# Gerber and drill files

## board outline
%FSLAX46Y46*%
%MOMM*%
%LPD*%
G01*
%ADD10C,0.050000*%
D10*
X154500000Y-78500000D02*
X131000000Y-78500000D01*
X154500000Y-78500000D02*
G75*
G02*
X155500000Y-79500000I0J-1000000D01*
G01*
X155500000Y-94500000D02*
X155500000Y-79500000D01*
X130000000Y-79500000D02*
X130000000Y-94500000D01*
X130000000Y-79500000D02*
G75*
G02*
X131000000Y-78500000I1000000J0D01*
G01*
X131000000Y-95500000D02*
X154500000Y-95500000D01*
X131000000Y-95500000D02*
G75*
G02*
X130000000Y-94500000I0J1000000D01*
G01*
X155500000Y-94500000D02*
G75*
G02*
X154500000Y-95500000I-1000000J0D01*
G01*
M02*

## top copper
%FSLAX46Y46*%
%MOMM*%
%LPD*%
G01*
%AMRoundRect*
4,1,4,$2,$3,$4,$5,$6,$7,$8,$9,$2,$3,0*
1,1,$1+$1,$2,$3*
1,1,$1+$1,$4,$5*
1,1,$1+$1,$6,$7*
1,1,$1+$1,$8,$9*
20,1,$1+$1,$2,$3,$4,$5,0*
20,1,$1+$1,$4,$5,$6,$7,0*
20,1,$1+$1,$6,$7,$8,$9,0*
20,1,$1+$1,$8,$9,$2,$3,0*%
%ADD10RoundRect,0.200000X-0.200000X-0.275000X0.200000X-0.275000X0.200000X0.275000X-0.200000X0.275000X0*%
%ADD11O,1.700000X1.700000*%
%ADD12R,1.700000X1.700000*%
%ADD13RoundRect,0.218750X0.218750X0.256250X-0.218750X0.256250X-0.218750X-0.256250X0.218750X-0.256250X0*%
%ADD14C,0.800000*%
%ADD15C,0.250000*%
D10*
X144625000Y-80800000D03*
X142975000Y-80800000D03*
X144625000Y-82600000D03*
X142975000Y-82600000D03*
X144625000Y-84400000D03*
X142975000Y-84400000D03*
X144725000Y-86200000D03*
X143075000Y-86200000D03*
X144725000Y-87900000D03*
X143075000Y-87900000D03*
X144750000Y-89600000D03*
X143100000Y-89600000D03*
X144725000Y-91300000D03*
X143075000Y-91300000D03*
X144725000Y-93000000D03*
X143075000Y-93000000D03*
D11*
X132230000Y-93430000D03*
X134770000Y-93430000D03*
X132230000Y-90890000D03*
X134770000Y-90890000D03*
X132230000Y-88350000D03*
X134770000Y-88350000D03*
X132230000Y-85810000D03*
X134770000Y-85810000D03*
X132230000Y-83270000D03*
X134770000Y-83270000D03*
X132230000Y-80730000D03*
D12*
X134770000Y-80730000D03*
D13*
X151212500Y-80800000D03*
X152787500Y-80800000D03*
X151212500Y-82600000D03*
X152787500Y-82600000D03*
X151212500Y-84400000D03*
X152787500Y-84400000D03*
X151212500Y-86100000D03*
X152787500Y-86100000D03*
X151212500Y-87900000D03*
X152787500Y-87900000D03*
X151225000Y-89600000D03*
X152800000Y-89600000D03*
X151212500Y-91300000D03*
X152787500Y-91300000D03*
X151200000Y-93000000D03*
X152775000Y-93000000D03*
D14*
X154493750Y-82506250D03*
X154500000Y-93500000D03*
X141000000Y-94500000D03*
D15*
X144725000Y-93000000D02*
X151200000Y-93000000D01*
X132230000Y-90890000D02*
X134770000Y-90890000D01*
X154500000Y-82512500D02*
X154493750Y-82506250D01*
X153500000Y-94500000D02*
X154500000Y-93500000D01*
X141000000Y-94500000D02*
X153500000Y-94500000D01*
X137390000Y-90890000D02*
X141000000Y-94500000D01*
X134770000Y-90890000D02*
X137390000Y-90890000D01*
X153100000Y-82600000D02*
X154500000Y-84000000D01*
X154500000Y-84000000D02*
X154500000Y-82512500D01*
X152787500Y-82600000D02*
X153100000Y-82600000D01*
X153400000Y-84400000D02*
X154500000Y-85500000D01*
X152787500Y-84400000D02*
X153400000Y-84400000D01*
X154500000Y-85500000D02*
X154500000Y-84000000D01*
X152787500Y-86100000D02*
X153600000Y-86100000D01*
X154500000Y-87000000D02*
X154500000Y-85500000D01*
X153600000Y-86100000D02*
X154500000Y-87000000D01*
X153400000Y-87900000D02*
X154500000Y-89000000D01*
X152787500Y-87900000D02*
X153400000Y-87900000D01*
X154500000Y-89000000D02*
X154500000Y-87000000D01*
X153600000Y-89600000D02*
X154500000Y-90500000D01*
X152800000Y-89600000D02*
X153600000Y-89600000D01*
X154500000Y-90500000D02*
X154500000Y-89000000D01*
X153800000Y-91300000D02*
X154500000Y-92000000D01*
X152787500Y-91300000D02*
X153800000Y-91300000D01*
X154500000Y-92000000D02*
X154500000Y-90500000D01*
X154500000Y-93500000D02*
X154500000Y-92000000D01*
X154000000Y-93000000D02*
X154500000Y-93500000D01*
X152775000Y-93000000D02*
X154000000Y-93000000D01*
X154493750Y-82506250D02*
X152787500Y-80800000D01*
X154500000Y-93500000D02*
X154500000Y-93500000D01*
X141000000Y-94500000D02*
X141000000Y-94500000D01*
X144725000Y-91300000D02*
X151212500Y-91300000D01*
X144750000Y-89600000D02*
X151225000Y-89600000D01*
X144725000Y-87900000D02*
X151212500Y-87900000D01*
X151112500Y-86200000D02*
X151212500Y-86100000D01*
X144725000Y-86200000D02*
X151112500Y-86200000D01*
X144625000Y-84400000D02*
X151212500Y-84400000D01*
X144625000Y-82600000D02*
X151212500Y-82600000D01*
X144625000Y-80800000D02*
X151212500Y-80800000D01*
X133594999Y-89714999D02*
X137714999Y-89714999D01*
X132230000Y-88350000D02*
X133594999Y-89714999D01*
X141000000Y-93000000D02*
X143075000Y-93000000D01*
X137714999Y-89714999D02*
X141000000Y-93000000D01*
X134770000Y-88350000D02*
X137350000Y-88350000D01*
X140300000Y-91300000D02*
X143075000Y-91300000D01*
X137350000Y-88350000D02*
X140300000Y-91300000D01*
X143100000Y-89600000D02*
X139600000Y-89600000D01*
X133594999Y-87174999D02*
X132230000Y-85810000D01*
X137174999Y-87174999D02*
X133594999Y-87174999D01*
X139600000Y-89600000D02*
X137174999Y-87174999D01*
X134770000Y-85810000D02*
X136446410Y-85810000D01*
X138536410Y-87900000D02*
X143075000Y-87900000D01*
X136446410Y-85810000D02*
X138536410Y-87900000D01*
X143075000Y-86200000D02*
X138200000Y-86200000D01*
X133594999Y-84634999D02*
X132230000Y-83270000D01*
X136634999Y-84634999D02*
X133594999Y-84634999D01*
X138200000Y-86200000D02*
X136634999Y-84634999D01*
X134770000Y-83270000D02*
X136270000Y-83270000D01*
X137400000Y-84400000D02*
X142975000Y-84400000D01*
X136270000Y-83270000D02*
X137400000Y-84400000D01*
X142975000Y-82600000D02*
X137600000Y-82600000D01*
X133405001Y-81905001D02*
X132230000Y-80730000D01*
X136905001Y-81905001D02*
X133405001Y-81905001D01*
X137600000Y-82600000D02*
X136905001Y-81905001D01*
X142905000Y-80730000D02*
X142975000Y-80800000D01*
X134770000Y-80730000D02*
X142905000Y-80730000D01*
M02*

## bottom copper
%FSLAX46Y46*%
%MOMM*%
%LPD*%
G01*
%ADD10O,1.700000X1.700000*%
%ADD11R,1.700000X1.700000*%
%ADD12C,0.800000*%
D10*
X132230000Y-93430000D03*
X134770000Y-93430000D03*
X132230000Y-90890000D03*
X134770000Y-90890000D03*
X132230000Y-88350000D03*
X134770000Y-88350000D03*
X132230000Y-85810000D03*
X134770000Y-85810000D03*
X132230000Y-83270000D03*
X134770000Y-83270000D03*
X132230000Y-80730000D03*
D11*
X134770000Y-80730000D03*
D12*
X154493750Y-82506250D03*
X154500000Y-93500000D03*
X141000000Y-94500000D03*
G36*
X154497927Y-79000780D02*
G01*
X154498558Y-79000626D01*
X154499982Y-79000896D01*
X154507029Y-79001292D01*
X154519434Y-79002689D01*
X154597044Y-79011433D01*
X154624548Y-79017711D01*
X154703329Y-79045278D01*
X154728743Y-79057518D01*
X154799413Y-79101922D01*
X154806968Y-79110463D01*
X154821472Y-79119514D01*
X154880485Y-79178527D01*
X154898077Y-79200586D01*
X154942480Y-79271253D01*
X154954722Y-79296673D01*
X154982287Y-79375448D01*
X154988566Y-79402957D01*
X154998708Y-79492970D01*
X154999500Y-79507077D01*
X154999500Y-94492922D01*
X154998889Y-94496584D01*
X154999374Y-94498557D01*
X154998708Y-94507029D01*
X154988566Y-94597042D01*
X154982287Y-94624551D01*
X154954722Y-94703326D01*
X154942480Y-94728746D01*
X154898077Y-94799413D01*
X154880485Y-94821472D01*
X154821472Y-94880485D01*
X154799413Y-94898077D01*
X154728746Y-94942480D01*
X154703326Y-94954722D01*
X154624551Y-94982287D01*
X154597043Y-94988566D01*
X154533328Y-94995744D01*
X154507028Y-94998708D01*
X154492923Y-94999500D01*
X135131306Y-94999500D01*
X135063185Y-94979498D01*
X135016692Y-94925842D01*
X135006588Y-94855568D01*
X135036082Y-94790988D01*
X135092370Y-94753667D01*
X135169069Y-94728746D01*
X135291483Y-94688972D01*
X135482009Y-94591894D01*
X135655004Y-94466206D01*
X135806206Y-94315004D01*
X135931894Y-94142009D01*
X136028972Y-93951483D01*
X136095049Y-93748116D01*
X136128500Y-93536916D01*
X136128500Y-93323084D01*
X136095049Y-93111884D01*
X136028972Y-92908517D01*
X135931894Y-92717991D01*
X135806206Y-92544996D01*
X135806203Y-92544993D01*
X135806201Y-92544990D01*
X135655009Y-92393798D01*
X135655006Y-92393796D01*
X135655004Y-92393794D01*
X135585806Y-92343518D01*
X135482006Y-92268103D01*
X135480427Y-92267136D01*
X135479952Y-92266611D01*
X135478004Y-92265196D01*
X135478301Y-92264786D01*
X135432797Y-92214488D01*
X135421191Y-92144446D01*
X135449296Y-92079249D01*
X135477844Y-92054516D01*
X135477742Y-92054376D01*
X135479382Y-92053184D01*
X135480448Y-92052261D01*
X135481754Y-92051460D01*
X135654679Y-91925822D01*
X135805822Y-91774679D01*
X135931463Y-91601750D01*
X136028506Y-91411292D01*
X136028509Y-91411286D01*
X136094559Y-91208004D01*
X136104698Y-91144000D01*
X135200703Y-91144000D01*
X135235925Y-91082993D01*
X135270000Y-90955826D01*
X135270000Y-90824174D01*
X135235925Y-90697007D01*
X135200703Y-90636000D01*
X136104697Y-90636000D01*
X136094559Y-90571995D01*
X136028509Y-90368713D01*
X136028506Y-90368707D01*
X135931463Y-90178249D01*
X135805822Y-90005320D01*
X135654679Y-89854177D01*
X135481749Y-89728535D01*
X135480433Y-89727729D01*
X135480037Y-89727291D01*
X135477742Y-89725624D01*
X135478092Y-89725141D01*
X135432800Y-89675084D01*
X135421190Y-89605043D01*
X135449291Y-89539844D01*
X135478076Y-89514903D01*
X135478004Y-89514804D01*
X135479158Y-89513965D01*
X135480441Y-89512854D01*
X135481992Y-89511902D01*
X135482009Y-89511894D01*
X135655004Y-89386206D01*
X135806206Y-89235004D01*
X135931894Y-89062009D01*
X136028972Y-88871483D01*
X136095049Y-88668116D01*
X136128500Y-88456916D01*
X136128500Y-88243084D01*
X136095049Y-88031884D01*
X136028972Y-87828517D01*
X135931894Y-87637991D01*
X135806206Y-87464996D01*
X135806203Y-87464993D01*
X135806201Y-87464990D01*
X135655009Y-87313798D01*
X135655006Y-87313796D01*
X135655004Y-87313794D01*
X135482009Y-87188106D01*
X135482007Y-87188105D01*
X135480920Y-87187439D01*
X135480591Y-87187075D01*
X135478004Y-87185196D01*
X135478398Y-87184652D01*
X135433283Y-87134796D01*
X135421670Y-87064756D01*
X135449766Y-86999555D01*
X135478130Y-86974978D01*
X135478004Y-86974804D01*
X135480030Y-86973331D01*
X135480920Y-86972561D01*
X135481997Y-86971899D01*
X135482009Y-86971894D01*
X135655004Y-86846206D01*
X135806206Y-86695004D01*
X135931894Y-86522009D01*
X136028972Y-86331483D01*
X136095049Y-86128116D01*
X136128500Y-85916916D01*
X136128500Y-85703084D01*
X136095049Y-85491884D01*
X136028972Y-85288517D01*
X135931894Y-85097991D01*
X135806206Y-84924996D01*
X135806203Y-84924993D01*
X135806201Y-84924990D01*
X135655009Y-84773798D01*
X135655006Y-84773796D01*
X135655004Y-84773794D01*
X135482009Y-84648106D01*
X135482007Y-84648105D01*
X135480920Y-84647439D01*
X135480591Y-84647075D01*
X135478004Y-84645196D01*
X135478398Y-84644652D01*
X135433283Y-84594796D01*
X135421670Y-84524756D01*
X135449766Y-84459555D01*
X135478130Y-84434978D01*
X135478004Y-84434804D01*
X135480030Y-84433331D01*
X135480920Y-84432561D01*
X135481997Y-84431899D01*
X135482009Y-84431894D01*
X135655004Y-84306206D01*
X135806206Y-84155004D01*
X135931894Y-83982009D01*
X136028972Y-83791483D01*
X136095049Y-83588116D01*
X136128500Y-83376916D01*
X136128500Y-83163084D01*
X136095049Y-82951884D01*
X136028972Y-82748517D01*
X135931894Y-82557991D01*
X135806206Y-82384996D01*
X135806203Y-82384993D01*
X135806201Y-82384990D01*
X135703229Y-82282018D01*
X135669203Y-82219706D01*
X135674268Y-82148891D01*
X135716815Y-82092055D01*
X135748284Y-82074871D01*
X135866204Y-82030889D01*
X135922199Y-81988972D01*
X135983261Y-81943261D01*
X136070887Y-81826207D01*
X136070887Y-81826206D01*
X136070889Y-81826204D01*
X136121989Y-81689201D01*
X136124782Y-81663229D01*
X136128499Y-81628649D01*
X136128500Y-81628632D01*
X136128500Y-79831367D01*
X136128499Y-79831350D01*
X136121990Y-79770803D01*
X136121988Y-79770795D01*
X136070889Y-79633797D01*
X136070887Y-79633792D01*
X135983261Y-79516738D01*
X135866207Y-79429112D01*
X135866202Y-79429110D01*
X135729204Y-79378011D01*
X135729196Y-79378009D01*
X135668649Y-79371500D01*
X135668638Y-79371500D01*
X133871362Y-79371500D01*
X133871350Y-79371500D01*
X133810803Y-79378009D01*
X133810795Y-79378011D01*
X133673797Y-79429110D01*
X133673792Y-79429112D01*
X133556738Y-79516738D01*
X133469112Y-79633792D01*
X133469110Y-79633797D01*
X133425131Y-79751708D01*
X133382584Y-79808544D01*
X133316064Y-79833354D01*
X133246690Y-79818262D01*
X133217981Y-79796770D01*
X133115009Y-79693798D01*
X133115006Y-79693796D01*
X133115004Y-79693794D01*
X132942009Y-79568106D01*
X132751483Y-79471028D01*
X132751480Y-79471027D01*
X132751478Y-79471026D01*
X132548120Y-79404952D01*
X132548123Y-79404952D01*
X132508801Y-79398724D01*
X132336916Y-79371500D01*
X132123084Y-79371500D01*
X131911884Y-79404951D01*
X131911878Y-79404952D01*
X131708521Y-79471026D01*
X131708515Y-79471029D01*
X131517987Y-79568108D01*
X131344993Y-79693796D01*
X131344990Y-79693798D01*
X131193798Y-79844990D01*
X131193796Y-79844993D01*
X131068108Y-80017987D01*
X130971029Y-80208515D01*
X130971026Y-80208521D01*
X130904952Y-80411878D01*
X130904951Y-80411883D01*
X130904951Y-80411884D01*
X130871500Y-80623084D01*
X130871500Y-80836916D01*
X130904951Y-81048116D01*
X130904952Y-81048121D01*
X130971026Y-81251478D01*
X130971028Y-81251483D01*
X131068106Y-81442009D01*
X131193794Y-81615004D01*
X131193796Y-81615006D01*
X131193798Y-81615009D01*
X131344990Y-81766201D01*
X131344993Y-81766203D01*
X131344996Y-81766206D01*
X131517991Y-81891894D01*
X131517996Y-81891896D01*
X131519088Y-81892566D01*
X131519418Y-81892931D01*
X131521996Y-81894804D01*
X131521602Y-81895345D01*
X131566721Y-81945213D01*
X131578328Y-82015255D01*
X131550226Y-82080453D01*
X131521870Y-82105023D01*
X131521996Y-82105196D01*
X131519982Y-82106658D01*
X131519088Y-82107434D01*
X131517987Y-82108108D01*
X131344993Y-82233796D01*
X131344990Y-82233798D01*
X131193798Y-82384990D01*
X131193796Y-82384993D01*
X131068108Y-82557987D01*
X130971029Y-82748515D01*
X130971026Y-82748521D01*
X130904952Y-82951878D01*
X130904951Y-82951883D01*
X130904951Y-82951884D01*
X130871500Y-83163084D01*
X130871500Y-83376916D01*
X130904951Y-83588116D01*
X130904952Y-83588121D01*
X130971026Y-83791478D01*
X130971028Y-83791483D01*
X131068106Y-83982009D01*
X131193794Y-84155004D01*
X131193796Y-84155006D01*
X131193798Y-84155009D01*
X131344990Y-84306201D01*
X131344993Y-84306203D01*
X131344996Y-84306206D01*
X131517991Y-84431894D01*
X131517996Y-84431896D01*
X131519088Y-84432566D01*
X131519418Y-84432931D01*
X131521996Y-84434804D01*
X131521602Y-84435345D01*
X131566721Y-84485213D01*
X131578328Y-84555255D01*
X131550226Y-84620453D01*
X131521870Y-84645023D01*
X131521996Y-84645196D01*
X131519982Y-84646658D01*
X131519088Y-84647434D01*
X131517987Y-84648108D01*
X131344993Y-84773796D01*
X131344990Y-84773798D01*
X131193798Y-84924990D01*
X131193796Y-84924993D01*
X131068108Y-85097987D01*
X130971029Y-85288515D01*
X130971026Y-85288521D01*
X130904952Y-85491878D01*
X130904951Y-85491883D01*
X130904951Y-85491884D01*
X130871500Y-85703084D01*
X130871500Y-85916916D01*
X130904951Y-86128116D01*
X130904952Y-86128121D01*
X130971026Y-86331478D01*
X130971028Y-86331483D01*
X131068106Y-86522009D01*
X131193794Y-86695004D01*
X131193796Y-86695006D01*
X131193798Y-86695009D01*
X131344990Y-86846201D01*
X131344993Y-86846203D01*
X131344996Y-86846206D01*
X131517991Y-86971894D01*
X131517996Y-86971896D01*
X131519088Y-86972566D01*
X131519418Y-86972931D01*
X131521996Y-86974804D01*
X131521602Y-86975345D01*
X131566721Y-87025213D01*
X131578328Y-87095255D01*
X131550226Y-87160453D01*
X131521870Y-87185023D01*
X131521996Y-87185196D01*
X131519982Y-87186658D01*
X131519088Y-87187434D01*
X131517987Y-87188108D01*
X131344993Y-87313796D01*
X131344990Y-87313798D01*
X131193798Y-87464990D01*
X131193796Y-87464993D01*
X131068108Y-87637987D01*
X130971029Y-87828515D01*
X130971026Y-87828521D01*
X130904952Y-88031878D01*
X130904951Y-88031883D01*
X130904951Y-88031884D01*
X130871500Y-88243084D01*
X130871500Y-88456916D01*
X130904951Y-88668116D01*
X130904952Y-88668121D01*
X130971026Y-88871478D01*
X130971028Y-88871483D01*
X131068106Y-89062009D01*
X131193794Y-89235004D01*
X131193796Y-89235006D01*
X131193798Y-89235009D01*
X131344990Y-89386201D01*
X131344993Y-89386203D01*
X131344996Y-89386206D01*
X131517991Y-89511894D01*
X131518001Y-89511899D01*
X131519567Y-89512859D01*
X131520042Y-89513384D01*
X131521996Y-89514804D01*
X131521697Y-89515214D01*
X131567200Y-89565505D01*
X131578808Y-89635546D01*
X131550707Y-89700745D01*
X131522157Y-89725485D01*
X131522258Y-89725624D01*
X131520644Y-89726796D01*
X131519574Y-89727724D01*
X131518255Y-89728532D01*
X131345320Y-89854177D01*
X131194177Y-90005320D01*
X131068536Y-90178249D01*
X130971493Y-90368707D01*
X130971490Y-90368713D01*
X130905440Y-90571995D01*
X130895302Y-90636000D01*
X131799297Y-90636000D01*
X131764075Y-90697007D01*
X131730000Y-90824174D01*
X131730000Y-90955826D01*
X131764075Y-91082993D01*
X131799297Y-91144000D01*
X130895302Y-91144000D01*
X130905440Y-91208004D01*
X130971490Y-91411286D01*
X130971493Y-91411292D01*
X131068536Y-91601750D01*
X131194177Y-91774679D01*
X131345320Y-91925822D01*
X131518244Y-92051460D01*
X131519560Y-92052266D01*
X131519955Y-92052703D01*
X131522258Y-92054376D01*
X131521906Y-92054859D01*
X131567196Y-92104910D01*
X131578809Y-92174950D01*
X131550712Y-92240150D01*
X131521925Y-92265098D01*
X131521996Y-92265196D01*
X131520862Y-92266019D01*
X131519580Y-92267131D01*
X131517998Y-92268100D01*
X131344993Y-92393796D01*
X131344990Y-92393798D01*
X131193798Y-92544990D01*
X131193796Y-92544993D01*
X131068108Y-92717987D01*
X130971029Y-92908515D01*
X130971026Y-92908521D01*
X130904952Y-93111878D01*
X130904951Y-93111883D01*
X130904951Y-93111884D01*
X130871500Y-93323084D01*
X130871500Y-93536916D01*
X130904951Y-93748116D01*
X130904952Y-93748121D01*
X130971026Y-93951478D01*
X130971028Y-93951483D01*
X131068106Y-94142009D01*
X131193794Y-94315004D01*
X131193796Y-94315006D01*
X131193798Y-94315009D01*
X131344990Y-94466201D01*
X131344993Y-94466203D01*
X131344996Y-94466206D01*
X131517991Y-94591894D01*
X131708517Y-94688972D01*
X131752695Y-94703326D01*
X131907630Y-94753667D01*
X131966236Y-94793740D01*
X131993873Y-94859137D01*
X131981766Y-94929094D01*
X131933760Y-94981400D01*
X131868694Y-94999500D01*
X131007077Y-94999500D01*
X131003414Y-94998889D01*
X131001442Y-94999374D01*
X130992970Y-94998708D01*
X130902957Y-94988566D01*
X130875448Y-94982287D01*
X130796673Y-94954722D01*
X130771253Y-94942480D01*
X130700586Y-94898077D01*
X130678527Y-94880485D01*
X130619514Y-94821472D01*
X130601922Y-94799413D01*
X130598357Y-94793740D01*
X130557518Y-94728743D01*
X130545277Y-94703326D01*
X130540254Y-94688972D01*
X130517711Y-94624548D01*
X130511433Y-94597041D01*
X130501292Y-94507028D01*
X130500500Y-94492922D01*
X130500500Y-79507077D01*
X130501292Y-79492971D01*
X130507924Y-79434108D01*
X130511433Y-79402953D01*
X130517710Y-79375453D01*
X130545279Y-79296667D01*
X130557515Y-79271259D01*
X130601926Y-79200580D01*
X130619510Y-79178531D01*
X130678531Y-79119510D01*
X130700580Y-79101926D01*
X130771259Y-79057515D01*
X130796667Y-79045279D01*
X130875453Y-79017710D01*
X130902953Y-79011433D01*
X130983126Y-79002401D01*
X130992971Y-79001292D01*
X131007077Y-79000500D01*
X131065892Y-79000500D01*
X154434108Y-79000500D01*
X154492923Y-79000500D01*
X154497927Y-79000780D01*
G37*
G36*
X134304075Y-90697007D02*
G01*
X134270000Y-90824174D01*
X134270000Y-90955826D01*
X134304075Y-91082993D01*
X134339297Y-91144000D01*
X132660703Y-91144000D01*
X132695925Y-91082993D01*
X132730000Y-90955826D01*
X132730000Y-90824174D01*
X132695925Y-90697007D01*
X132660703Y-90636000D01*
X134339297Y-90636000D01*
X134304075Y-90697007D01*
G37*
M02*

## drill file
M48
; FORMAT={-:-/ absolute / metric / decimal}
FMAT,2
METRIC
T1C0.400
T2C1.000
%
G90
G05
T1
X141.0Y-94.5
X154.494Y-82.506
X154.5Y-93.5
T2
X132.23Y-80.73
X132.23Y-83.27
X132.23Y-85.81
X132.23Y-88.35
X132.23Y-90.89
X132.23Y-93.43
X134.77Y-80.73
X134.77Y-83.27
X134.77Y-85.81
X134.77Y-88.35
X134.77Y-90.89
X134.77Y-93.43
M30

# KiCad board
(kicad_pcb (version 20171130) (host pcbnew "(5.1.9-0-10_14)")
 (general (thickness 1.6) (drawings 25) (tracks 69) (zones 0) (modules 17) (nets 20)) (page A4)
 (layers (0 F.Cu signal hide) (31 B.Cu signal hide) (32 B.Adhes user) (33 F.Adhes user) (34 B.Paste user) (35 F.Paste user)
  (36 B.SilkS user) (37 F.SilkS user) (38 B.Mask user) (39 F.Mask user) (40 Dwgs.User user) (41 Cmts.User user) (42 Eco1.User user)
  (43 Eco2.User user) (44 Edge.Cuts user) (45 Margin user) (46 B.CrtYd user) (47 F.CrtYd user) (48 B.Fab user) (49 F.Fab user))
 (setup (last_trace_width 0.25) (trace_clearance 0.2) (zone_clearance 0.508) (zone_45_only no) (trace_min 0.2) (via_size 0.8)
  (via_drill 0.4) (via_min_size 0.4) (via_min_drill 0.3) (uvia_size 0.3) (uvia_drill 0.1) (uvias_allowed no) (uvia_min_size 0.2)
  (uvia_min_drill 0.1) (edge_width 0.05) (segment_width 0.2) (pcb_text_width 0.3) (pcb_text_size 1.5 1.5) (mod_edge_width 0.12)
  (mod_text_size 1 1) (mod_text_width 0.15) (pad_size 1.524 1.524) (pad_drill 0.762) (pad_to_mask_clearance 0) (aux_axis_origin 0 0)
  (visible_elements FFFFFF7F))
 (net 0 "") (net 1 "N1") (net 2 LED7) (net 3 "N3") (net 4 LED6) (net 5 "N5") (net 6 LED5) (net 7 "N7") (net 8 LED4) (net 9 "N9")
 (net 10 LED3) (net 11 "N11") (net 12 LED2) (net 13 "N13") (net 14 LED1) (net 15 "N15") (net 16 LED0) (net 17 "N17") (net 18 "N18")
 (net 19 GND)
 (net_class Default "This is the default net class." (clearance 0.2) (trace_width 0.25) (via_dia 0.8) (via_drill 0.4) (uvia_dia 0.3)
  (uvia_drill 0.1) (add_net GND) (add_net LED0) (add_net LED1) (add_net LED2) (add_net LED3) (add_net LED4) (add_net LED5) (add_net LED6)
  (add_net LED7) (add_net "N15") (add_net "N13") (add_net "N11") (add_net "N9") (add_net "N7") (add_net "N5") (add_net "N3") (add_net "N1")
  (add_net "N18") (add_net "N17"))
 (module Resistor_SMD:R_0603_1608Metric (layer F.Cu) (at 143.8 80.8)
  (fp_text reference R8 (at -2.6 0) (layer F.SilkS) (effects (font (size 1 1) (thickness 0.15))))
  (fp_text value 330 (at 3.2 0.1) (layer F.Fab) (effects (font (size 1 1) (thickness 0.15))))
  (pad 2 smd roundrect (at 0.825 0) (size 0.8 0.95) (layers F.Cu F.Paste F.Mask) (roundrect_rratio 0.25) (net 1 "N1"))
  (pad 1 smd roundrect (at -0.825 0) (size 0.8 0.95) (layers F.Cu F.Paste F.Mask) (roundrect_rratio 0.25) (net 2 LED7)))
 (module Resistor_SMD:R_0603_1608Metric (layer F.Cu) (at 143.8 82.6)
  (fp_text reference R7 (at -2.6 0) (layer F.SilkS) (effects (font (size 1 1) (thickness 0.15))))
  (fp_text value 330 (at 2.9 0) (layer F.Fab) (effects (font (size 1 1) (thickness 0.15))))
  (pad 2 smd roundrect (at 0.825 0) (size 0.8 0.95) (layers F.Cu F.Paste F.Mask) (roundrect_rratio 0.25) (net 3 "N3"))
  (pad 1 smd roundrect (at -0.825 0) (size 0.8 0.95) (layers F.Cu F.Paste F.Mask) (roundrect_rratio 0.25) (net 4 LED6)))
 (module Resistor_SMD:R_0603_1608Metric (layer F.Cu) (at 143.8 84.4)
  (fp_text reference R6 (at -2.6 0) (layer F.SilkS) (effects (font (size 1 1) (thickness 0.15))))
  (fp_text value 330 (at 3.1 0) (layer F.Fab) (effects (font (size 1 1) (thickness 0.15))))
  (pad 2 smd roundrect (at 0.825 0) (size 0.8 0.95) (layers F.Cu F.Paste F.Mask) (roundrect_rratio 0.25) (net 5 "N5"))
  (pad 1 smd roundrect (at -0.825 0) (size 0.8 0.95) (layers F.Cu F.Paste F.Mask) (roundrect_rratio 0.25) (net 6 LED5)))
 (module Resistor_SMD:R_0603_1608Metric (layer F.Cu) (at 143.9 86.2)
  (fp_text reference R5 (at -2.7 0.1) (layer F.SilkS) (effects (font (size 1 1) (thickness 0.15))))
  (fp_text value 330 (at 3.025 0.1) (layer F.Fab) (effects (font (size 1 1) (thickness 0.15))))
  (pad 2 smd roundrect (at 0.825 0) (size 0.8 0.95) (layers F.Cu F.Paste F.Mask) (roundrect_rratio 0.25) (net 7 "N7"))
  (pad 1 smd roundrect (at -0.825 0) (size 0.8 0.95) (layers F.Cu F.Paste F.Mask) (roundrect_rratio 0.25) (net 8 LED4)))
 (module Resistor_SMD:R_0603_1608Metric (layer F.Cu) (at 143.9 87.9)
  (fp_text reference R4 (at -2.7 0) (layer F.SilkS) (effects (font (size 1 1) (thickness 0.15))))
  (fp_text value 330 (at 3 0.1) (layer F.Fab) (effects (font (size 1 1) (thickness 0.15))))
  (pad 2 smd roundrect (at 0.825 0) (size 0.8 0.95) (layers F.Cu F.Paste F.Mask) (roundrect_rratio 0.25) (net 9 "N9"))
  (pad 1 smd roundrect (at -0.825 0) (size 0.8 0.95) (layers F.Cu F.Paste F.Mask) (roundrect_rratio 0.25) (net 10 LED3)))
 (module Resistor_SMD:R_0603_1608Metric (layer F.Cu) (at 143.925 89.6)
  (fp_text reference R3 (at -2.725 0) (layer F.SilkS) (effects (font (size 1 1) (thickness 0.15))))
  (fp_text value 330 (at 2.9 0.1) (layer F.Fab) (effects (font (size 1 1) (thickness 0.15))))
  (pad 2 smd roundrect (at 0.825 0) (size 0.8 0.95) (layers F.Cu F.Paste F.Mask) (roundrect_rratio 0.25) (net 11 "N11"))
  (pad 1 smd roundrect (at -0.825 0) (size 0.8 0.95) (layers F.Cu F.Paste F.Mask) (roundrect_rratio 0.25) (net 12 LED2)))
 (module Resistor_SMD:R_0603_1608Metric (layer F.Cu) (at 143.9 91.3)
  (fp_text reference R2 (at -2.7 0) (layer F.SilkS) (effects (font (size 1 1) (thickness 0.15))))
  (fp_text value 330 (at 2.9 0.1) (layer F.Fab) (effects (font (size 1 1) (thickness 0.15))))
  (pad 2 smd roundrect (at 0.825 0) (size 0.8 0.95) (layers F.Cu F.Paste F.Mask) (roundrect_rratio 0.25) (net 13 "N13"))
  (pad 1 smd roundrect (at -0.825 0) (size 0.8 0.95) (layers F.Cu F.Paste F.Mask) (roundrect_rratio 0.25) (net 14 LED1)))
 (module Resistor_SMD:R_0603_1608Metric (layer F.Cu) (at 143.9 93)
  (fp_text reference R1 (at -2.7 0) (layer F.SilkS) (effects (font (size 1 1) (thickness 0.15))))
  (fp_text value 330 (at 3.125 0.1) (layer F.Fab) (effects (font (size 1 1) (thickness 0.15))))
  (pad 2 smd roundrect (at 0.825 0) (size 0.8 0.95) (layers F.Cu F.Paste F.Mask) (roundrect_rratio 0.25) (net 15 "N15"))
  (pad 1 smd roundrect (at -0.825 0) (size 0.8 0.95) (layers F.Cu F.Paste F.Mask) (roundrect_rratio 0.25) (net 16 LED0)))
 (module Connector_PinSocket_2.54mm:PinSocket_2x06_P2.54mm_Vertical (layer F.Cu) (at 134.77 80.73)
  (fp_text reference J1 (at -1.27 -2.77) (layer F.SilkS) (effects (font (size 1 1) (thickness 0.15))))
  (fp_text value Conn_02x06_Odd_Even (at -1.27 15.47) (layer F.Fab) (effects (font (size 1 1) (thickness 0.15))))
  (pad 12 thru_hole oval (at -2.54 12.7) (size 1.7 1.7) (drill 1) (layers *.Cu *.Mask) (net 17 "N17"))
  (pad 11 thru_hole oval (at 0 12.7) (size 1.7 1.7) (drill 1) (layers *.Cu *.Mask) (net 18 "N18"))
  (pad 10 thru_hole oval (at -2.54 10.16) (size 1.7 1.7) (drill 1) (layers *.Cu *.Mask) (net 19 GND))
  (pad 9 thru_hole oval (at 0 10.16) (size 1.7 1.7) (drill 1) (layers *.Cu *.Mask) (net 19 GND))
  (pad 8 thru_hole oval (at -2.54 7.62) (size 1.7 1.7) (drill 1) (layers *.Cu *.Mask) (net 16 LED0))
  (pad 7 thru_hole oval (at 0 7.62) (size 1.7 1.7) (drill 1) (layers *.Cu *.Mask) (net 14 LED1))
  (pad 6 thru_hole oval (at -2.54 5.08) (size 1.7 1.7) (drill 1) (layers *.Cu *.Mask) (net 12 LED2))
  (pad 5 thru_hole oval (at 0 5.08) (size 1.7 1.7) (drill 1) (layers *.Cu *.Mask) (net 10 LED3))
  (pad 4 thru_hole oval (at -2.54 2.54) (size 1.7 1.7) (drill 1) (layers *.Cu *.Mask) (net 8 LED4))
  (pad 3 thru_hole oval (at 0 2.54) (size 1.7 1.7) (drill 1) (layers *.Cu *.Mask) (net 6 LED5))
  (pad 2 thru_hole oval (at -2.54 0) (size 1.7 1.7) (drill 1) (layers *.Cu *.Mask) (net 4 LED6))
  (pad 1 thru_hole rect (at 0 0) (size 1.7 1.7) (drill 1) (layers *.Cu *.Mask) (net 2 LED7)))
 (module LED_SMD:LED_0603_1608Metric (layer F.Cu) (at 152 80.8 180)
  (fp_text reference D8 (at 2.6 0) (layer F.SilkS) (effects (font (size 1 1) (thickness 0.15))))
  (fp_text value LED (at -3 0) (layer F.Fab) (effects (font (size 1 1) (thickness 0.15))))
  (pad 2 smd roundrect (at 0.7875 0 180) (size 0.875 0.95) (layers F.Cu F.Paste F.Mask) (roundrect_rratio 0.25) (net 1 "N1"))
  (pad 1 smd roundrect (at -0.7875 0 180) (size 0.875 0.95) (layers F.Cu F.Paste F.Mask) (roundrect_rratio 0.25) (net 19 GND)))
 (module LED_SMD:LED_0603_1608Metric (layer F.Cu) (at 152 82.6 180)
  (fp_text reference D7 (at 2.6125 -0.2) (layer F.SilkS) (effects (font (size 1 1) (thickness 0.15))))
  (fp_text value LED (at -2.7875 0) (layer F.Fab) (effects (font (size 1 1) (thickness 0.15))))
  (pad 2 smd roundrect (at 0.7875 0 180) (size 0.875 0.95) (layers F.Cu F.Paste F.Mask) (roundrect_rratio 0.25) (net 3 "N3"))
  (pad 1 smd roundrect (at -0.7875 0 180) (size 0.875 0.95) (layers F.Cu F.Paste F.Mask) (roundrect_rratio 0.25) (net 19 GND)))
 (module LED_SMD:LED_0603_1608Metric (layer F.Cu) (at 152 84.4 180)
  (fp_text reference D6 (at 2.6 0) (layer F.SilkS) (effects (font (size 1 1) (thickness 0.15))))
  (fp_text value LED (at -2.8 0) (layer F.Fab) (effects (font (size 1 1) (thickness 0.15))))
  (pad 2 smd roundrect (at 0.7875 0 180) (size 0.875 0.95) (layers F.Cu F.Paste F.Mask) (roundrect_rratio 0.25) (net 5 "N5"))
  (pad 1 smd roundrect (at -0.7875 0 180) (size 0.875 0.95) (layers F.Cu F.Paste F.Mask) (roundrect_rratio 0.25) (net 19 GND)))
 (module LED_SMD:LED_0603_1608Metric (layer F.Cu) (at 152 86.1 180)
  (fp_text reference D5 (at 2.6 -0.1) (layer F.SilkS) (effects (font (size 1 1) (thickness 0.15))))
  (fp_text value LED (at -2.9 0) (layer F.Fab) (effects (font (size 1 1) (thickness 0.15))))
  (pad 2 smd roundrect (at 0.7875 0 180) (size 0.875 0.95) (layers F.Cu F.Paste F.Mask) (roundrect_rratio 0.25) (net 7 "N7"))
  (pad 1 smd roundrect (at -0.7875 0 180) (size 0.875 0.95) (layers F.Cu F.Paste F.Mask) (roundrect_rratio 0.25) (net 19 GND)))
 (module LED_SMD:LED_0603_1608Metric (layer F.Cu) (at 152 87.9 180)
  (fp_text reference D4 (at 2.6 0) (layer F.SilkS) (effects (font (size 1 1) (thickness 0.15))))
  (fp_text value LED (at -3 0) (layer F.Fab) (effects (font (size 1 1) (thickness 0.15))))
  (pad 2 smd roundrect (at 0.7875 0 180) (size 0.875 0.95) (layers F.Cu F.Paste F.Mask) (roundrect_rratio 0.25) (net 9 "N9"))
  (pad 1 smd roundrect (at -0.7875 0 180) (size 0.875 0.95) (layers F.Cu F.Paste F.Mask) (roundrect_rratio 0.25) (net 19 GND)))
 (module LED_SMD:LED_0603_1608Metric (layer F.Cu) (at 152.0125 89.6 180)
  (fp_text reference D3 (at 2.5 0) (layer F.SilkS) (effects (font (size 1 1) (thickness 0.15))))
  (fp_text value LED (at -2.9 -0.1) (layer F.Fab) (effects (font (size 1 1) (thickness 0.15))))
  (pad 2 smd roundrect (at 0.7875 0 180) (size 0.875 0.95) (layers F.Cu F.Paste F.Mask) (roundrect_rratio 0.25) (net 11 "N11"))
  (pad 1 smd roundrect (at -0.7875 0 180) (size 0.875 0.95) (layers F.Cu F.Paste F.Mask) (roundrect_rratio 0.25) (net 19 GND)))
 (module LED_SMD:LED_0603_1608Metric (layer F.Cu) (at 152 91.3 180)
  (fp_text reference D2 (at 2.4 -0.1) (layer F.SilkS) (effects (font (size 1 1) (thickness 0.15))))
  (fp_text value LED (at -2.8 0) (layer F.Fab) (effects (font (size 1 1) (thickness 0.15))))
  (pad 2 smd roundrect (at 0.7875 0 180) (size 0.875 0.95) (layers F.Cu F.Paste F.Mask) (roundrect_rratio 0.25) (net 13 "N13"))
  (pad 1 smd roundrect (at -0.7875 0 180) (size 0.875 0.95) (layers F.Cu F.Paste F.Mask) (roundrect_rratio 0.25) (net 19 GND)))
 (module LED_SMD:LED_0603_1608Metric (layer F.Cu) (at 151.9875 93 180)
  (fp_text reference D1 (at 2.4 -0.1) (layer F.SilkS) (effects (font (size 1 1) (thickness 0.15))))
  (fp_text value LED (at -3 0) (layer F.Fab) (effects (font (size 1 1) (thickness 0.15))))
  (pad 2 smd roundrect (at 0.7875 0 180) (size 0.875 0.95) (layers F.Cu F.Paste F.Mask) (roundrect_rratio 0.25) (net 15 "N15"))
  (pad 1 smd roundrect (at -0.7875 0 180) (size 0.875 0.95) (layers F.Cu F.Paste F.Mask) (roundrect_rratio 0.25) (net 19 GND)))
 (gr_line (start 154.5 78.5) (end 131 78.5) (layer Edge.Cuts) (width 0.05))
 (gr_arc (start 154.5 79.5) (end 155.5 79.5) (angle -90) (layer Edge.Cuts) (width 0.05))
 (gr_line (start 155.5 94.5) (end 155.5 79.5) (layer Edge.Cuts) (width 0.05))
 (gr_line (start 130 79.5) (end 130 94.5) (layer Edge.Cuts) (width 0.05))
 (gr_arc (start 131 79.5) (end 131 78.5) (angle -90) (layer Edge.Cuts) (width 0.05))
 (gr_line (start 131 95.5) (end 154.5 95.5) (layer Edge.Cuts) (width 0.05))
 (gr_arc (start 131 94.5) (end 130 94.5) (angle -90) (layer Edge.Cuts) (width 0.05))
 (gr_arc (start 154.5 94.5) (end 154.5 95.5) (angle -90) (layer Edge.Cuts) (width 0.05))
 (segment (start 144.725 93) (end 151.2 93) (width 0.25) (layer F.Cu) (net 15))
 (segment (start 132.23 90.89) (end 134.77 90.89) (width 0.25) (layer F.Cu) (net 19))
 (segment (start 154.5 82.5125) (end 154.49375 82.50625) (width 0.25) (layer F.Cu) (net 19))
 (segment (start 153.5 94.5) (end 154.5 93.5) (width 0.25) (layer F.Cu) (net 19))
 (segment (start 141 94.5) (end 153.5 94.5) (width 0.25) (layer F.Cu) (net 19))
 (segment (start 137.39 90.89) (end 141 94.5) (width 0.25) (layer F.Cu) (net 19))
 (segment (start 134.77 90.89) (end 137.39 90.89) (width 0.25) (layer F.Cu) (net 19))
 (segment (start 153.1 82.6) (end 154.5 84) (width 0.25) (layer F.Cu) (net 19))
 (segment (start 154.5 84) (end 154.5 82.5125) (width 0.25) (layer F.Cu) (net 19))
 (segment (start 152.7875 82.6) (end 153.1 82.6) (width 0.25) (layer F.Cu) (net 19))
 (segment (start 153.4 84.4) (end 154.5 85.5) (width 0.25) (layer F.Cu) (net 19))
 (segment (start 152.7875 84.4) (end 153.4 84.4) (width 0.25) (layer F.Cu) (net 19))
 (segment (start 154.5 85.5) (end 154.5 84) (width 0.25) (layer F.Cu) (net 19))
 (segment (start 152.7875 86.1) (end 153.6 86.1) (width 0.25) (layer F.Cu) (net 19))
 (segment (start 154.5 87) (end 154.5 85.5) (width 0.25) (layer F.Cu) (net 19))
 (segment (start 153.6 86.1) (end 154.5 87) (width 0.25) (layer F.Cu) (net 19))
 (segment (start 153.4 87.9) (end 154.5 89) (width 0.25) (layer F.Cu) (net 19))
 (segment (start 152.7875 87.9) (end 153.4 87.9) (width 0.25) (layer F.Cu) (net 19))
 (segment (start 154.5 89) (end 154.5 87) (width 0.25) (layer F.Cu) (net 19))
 (segment (start 153.6 89.6) (end 154.5 90.5) (width 0.25) (layer F.Cu) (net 19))
 (segment (start 152.8 89.6) (end 153.6 89.6) (width 0.25) (layer F.Cu) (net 19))
 (segment (start 154.5 90.5) (end 154.5 89) (width 0.25) (layer F.Cu) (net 19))
 (segment (start 153.8 91.3) (end 154.5 92) (width 0.25) (layer F.Cu) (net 19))
 (segment (start 152.7875 91.3) (end 153.8 91.3) (width 0.25) (layer F.Cu) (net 19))
 (segment (start 154.5 92) (end 154.5 90.5) (width 0.25) (layer F.Cu) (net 19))
 (segment (start 154.5 93.5) (end 154.5 92) (width 0.25) (layer F.Cu) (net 19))
 (segment (start 154 93) (end 154.5 93.5) (width 0.25) (layer F.Cu) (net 19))
 (segment (start 152.775 93) (end 154 93) (width 0.25) (layer F.Cu) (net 19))
 (segment (start 154.49375 82.50625) (end 152.7875 80.8) (width 0.25) (layer F.Cu) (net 19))
 (via (at 154.49375 82.50625) (size 0.8) (drill 0.4) (layers F.Cu B.Cu) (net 19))
 (segment (start 154.5 93.5) (end 154.5 93.5) (width 0.25) (layer F.Cu) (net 19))
 (via (at 154.5 93.5) (size 0.8) (drill 0.4) (layers F.Cu B.Cu) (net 19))
 (segment (start 141 94.5) (end 141 94.5) (width 0.25) (layer F.Cu) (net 19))
 (via (at 141 94.5) (size 0.8) (drill 0.4) (layers F.Cu B.Cu) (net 19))
 (segment (start 144.725 91.3) (end 151.2125 91.3) (width 0.25) (layer F.Cu) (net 13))
 (segment (start 144.75 89.6) (end 151.225 89.6) (width 0.25) (layer F.Cu) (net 11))
 (segment (start 144.725 87.9) (end 151.2125 87.9) (width 0.25) (layer F.Cu) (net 9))
 (segment (start 151.1125 86.2) (end 151.2125 86.1) (width 0.25) (layer F.Cu) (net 7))
 (segment (start 144.725 86.2) (end 151.1125 86.2) (width 0.25) (layer F.Cu) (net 7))
 (segment (start 144.625 84.4) (end 151.2125 84.4) (width 0.25) (layer F.Cu) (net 5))
 (segment (start 144.625 82.6) (end 151.2125 82.6) (width 0.25) (layer F.Cu) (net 3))
 (segment (start 144.625 80.8) (end 151.2125 80.8) (width 0.25) (layer F.Cu) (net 1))
 (segment (start 133.594999 89.714999) (end 137.714999 89.714999) (width 0.25) (layer F.Cu) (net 16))
 (segment (start 132.23 88.35) (end 133.594999 89.714999) (width 0.25) (layer F.Cu) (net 16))
 (segment (start 141 93) (end 143.075 93) (width 0.25) (layer F.Cu) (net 16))
 (segment (start 137.714999 89.714999) (end 141 93) (width 0.25) (layer F.Cu) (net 16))
 (segment (start 134.77 88.35) (end 137.35 88.35) (width 0.25) (layer F.Cu) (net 14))
 (segment (start 140.3 91.3) (end 143.075 91.3) (width 0.25) (layer F.Cu) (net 14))
 (segment (start 137.35 88.35) (end 140.3 91.3) (width 0.25) (layer F.Cu) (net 14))
 (segment (start 143.1 89.6) (end 139.6 89.6) (width 0.25) (layer F.Cu) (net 12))
 (segment (start 133.594999 87.174999) (end 132.23 85.81) (width 0.25) (layer F.Cu) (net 12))
 (segment (start 137.174999 87.174999) (end 133.594999 87.174999) (width 0.25) (layer F.Cu) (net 12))
 (segment (start 139.6 89.6) (end 137.174999 87.174999) (width 0.25) (layer F.Cu) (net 12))
 (segment (start 134.77 85.81) (end 136.44641 85.81) (width 0.25) (layer F.Cu) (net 10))
 (segment (start 138.53641 87.9) (end 143.075 87.9) (width 0.25) (layer F.Cu) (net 10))
 (segment (start 136.44641 85.81) (end 138.53641 87.9) (width 0.25) (layer F.Cu) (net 10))
 (segment (start 143.075 86.2) (end 138.2 86.2) (width 0.25) (layer F.Cu) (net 8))
 (segment (start 133.594999 84.634999) (end 132.23 83.27) (width 0.25) (layer F.Cu) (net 8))
 (segment (start 136.634999 84.634999) (end 133.594999 84.634999) (width 0.25) (layer F.Cu) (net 8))
 (segment (start 138.2 86.2) (end 136.634999 84.634999) (width 0.25) (layer F.Cu) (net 8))
 (segment (start 134.77 83.27) (end 136.27 83.27) (width 0.25) (layer F.Cu) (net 6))
 (segment (start 137.4 84.4) (end 142.975 84.4) (width 0.25) (layer F.Cu) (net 6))
 (segment (start 136.27 83.27) (end 137.4 84.4) (width 0.25) (layer F.Cu) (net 6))
 (segment (start 142.975 82.6) (end 137.6 82.6) (width 0.25) (layer F.Cu) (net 4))
 (segment (start 133.405001 81.905001) (end 132.23 80.73) (width 0.25) (layer F.Cu) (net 4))
 (segment (start 136.905001 81.905001) (end 133.405001 81.905001) (width 0.25) (layer F.Cu) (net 4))
 (segment (start 137.6 82.6) (end 136.905001 81.905001) (width 0.25) (layer F.Cu) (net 4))
 (segment (start 142.905 80.73) (end 142.975 80.8) (width 0.25) (layer F.Cu) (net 2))
 (segment (start 134.77 80.73) (end 142.905 80.73) (width 0.25) (layer F.Cu) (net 2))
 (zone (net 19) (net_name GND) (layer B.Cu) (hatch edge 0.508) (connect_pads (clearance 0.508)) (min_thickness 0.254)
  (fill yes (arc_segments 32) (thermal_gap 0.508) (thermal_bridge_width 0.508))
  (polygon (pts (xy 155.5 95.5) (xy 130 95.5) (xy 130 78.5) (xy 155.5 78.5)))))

